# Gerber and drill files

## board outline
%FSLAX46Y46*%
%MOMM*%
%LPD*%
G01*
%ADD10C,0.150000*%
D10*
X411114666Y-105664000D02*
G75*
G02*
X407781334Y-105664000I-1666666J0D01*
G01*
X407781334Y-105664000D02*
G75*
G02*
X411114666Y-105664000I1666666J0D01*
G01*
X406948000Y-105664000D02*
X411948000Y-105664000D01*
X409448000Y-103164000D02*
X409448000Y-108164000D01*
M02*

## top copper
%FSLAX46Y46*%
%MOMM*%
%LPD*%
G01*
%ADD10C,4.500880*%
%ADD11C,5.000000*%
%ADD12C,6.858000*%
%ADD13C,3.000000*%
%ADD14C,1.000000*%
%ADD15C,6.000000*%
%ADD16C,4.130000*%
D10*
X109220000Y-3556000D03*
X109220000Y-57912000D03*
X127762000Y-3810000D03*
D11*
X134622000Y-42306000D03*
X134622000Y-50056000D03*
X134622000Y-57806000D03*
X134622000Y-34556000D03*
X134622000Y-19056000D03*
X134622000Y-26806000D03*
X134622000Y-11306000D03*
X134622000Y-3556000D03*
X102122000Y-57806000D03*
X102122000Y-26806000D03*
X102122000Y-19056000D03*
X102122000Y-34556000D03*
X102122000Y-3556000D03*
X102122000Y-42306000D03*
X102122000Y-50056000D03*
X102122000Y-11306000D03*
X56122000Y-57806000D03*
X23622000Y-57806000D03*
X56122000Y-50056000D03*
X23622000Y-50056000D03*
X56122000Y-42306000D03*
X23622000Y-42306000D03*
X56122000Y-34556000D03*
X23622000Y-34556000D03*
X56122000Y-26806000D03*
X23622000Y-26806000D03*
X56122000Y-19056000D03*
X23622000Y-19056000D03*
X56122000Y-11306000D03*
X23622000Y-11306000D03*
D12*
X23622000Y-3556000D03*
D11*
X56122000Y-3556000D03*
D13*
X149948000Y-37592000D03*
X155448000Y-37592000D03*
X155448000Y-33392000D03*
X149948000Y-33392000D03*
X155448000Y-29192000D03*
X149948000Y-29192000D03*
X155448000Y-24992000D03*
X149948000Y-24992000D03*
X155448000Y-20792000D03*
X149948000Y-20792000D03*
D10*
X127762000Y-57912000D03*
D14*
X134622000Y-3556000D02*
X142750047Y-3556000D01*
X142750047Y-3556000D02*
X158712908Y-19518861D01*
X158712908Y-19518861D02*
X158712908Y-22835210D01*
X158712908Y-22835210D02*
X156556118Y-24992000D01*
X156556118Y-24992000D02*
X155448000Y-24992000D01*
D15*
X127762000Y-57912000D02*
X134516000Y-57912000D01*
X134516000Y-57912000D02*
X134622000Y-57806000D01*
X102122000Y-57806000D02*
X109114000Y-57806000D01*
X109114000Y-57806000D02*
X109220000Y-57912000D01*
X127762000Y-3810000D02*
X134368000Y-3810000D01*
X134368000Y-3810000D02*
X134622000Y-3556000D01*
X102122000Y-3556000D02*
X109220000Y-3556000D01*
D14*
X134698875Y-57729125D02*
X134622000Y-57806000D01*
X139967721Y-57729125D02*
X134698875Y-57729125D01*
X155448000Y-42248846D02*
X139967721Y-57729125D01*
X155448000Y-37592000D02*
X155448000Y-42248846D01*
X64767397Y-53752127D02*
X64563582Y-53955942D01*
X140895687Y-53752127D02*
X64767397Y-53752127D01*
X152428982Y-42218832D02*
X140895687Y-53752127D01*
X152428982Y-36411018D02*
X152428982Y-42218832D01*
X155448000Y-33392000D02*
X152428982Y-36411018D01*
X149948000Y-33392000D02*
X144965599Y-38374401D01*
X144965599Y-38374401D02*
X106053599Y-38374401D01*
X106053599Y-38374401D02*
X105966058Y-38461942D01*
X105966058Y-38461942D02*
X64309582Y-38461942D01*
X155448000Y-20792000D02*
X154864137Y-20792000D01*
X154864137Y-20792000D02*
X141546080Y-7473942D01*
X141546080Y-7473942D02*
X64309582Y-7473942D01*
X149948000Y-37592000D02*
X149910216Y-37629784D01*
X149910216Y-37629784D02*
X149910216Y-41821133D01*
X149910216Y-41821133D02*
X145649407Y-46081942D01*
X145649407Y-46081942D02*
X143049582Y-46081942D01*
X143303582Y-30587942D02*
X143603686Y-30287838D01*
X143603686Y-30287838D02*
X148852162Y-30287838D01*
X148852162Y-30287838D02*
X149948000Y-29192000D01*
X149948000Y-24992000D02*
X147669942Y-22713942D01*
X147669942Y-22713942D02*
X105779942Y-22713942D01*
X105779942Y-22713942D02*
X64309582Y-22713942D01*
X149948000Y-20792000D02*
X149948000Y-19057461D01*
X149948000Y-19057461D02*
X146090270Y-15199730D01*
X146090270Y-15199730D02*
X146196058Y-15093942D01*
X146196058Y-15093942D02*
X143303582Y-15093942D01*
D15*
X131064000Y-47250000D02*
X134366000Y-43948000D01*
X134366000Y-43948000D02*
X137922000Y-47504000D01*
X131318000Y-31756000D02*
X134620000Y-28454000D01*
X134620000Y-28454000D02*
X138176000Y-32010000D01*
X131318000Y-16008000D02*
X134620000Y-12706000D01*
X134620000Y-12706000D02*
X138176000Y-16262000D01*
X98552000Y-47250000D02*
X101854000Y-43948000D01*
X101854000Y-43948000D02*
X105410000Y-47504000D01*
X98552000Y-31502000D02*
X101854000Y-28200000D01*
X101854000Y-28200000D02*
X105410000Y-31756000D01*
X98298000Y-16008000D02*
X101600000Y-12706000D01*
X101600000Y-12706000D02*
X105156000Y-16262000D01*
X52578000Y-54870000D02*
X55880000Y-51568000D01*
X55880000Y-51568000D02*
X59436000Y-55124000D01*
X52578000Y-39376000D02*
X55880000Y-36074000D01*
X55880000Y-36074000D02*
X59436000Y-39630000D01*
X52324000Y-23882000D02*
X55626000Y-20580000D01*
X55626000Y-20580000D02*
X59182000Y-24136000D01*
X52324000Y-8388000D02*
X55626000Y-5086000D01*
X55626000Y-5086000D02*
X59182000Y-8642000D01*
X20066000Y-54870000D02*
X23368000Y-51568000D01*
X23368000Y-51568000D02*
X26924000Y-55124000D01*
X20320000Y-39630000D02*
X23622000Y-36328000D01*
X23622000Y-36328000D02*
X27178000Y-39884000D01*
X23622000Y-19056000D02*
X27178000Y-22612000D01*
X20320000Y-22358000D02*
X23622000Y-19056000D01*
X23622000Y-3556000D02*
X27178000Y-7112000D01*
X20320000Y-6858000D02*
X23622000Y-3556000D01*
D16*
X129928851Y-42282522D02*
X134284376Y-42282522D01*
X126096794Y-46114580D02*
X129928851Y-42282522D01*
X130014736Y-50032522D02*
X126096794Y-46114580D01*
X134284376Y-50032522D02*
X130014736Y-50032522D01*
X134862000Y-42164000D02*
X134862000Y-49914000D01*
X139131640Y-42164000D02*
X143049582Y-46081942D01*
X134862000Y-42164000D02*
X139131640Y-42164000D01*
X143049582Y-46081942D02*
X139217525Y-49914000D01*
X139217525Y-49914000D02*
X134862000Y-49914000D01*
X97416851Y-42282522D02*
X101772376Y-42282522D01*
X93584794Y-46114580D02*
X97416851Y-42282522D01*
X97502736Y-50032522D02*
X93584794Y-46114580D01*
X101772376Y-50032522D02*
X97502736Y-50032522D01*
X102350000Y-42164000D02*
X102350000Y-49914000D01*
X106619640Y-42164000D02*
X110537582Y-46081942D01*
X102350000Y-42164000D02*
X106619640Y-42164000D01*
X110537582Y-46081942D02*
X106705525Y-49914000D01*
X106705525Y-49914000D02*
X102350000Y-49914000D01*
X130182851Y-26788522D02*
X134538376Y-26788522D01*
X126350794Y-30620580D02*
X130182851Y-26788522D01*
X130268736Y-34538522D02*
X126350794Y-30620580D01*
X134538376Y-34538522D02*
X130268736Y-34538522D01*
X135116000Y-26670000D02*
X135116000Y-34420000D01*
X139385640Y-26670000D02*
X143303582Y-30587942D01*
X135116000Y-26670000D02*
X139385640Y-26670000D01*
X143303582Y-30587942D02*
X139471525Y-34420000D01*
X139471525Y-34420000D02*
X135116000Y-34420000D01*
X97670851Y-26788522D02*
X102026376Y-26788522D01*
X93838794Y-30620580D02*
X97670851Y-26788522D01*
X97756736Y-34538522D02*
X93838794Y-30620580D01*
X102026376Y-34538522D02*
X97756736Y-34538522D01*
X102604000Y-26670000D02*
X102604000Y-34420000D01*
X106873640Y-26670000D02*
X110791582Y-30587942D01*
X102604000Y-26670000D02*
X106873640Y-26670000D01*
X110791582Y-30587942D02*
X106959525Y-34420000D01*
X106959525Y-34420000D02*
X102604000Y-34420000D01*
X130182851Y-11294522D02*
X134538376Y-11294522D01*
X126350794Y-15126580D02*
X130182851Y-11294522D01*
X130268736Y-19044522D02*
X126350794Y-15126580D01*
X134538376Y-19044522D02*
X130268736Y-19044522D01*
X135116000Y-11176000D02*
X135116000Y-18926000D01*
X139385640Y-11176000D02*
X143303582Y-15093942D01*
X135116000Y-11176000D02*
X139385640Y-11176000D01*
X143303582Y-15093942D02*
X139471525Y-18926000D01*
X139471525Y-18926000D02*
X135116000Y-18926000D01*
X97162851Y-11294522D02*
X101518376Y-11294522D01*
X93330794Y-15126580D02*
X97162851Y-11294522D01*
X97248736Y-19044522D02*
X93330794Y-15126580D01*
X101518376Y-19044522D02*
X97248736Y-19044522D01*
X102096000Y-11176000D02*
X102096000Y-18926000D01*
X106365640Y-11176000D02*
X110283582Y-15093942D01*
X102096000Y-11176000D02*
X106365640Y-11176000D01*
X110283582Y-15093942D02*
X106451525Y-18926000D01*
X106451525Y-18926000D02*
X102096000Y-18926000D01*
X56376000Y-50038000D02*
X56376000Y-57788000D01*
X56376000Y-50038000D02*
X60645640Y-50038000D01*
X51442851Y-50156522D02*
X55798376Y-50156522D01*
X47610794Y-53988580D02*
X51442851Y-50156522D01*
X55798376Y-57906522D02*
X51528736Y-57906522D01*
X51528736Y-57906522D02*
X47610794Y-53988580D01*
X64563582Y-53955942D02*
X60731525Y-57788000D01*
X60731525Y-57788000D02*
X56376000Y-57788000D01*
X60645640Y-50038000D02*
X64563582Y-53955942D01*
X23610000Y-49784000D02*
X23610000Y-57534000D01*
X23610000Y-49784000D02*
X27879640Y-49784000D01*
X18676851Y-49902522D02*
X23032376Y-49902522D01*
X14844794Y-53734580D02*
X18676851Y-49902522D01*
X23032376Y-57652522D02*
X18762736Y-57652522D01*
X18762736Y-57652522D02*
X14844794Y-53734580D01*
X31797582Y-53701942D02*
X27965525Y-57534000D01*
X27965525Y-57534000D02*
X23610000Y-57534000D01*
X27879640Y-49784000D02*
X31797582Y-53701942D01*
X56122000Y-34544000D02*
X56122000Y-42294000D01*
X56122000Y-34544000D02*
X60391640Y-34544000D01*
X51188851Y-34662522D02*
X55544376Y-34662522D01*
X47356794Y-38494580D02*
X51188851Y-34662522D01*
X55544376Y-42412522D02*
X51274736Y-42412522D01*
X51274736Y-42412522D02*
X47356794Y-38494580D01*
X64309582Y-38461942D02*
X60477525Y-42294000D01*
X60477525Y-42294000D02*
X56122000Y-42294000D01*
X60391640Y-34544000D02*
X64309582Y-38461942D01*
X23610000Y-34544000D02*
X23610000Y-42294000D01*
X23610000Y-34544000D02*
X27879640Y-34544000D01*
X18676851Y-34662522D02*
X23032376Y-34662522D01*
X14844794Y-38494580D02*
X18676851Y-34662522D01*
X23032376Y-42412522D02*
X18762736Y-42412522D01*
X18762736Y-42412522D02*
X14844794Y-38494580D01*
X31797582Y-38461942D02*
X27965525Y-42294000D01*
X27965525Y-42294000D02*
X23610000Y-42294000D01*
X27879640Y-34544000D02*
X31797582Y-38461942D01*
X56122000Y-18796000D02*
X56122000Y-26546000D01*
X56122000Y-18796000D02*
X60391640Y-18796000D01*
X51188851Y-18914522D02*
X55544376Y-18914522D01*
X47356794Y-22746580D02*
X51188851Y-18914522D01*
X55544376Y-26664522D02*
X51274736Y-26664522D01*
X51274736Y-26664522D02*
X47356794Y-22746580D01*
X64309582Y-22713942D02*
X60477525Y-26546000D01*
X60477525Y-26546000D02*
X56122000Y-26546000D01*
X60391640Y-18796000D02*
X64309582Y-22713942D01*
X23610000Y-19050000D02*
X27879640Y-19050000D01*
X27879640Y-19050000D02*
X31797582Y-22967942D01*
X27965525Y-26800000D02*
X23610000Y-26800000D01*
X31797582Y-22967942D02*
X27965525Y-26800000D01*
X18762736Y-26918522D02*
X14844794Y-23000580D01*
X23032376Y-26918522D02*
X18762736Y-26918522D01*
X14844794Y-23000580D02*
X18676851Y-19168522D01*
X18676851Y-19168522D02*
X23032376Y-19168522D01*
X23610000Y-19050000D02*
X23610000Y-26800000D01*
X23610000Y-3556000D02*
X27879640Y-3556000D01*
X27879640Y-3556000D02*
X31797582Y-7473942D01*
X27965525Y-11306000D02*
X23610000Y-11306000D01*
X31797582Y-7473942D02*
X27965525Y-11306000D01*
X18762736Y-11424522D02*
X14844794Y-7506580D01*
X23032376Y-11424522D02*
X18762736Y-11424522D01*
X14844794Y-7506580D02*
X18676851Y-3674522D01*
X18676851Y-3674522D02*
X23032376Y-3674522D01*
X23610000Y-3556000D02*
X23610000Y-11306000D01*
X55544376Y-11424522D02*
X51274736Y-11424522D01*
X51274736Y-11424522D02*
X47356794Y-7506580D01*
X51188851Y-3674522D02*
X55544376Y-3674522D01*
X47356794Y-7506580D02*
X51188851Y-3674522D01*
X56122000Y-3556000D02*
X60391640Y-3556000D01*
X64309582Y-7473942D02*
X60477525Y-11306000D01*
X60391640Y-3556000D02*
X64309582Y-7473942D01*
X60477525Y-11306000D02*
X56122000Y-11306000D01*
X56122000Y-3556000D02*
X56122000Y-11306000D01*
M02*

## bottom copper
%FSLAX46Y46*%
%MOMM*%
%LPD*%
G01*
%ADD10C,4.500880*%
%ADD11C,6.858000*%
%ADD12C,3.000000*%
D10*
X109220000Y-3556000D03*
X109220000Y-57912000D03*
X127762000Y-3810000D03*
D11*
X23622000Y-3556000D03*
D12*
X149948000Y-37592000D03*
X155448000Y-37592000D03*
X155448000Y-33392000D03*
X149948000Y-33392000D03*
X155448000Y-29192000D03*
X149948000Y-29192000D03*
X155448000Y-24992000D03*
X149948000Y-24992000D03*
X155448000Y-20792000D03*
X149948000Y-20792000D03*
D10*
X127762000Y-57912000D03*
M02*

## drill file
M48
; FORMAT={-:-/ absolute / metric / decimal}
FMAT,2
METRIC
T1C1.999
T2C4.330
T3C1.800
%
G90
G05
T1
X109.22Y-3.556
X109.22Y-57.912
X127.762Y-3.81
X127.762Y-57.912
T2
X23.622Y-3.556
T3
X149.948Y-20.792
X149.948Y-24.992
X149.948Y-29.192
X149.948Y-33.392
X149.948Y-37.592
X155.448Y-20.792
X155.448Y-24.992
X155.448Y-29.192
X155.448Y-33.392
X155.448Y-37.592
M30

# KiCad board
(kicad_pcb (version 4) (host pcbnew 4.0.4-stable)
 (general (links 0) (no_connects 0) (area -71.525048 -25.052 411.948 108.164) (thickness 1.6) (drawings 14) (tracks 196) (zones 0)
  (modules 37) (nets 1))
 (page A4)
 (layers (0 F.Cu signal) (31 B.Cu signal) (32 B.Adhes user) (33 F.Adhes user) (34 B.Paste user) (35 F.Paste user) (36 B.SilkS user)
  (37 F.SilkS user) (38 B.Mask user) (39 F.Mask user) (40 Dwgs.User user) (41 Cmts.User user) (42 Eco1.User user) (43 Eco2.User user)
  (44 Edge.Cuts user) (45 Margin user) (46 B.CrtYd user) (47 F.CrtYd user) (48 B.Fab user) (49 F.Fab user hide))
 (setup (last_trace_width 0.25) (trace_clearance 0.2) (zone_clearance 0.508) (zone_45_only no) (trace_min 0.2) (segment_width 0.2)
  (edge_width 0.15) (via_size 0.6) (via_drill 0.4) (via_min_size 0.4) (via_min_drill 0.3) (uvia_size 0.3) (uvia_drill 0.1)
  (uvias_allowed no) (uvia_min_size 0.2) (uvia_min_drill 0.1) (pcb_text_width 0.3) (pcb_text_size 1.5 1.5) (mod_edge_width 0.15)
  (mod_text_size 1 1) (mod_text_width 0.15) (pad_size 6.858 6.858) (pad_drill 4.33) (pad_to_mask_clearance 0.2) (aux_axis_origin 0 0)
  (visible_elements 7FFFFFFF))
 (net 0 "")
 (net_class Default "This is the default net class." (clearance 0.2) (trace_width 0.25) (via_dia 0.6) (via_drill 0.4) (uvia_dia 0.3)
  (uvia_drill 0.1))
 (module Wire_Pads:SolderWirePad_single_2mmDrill (layer F.Cu) (at 109.22 3.556)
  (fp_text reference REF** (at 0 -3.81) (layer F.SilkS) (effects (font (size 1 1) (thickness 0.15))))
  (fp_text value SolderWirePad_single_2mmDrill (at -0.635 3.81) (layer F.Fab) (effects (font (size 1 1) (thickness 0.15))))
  (pad 1 thru_hole circle (at 0 0) (size 4.50088 4.50088) (drill 1.99898) (layers *.Cu *.Mask)))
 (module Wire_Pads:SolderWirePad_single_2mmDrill (layer F.Cu) (at 109.22 57.912)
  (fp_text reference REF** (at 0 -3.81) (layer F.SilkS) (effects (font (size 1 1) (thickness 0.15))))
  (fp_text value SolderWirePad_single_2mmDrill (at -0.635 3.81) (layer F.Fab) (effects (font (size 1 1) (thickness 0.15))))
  (pad 1 thru_hole circle (at 0 0) (size 4.50088 4.50088) (drill 1.99898) (layers *.Cu *.Mask)))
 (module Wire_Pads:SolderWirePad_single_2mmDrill (layer F.Cu) (at 127.762 3.81)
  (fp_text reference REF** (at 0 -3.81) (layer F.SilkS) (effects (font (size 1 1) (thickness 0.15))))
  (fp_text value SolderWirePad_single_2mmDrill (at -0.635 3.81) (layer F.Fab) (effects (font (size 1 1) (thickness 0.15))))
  (pad 1 thru_hole circle (at 0 0) (size 4.50088 4.50088) (drill 1.99898) (layers *.Cu *.Mask)))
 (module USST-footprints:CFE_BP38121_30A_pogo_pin (layer F.Cu) (at 174.5 53.736)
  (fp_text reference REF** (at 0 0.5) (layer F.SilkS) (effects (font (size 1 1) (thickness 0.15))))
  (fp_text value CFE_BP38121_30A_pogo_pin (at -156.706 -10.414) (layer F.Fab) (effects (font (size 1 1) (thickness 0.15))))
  (pad 6 smd circle (at -39.878 -11.43) (size 5 5) (layers F.Cu F.Paste F.Mask)))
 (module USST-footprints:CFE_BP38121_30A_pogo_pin (layer F.Cu) (at 174.5 61.486)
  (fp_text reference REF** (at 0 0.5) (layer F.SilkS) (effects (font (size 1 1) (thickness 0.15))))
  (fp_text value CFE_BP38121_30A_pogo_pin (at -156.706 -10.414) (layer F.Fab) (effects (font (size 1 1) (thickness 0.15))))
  (pad 7 smd circle (at -39.878 -11.43) (size 5 5) (layers F.Cu F.Paste F.Mask)))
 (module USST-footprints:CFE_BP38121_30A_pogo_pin (layer F.Cu) (at 174.5 69.236)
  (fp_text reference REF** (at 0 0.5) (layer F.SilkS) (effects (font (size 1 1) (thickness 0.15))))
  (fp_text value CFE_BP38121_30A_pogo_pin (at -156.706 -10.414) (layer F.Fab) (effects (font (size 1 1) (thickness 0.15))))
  (pad 8 smd circle (at -39.878 -11.43) (size 5 5) (layers F.Cu F.Paste F.Mask)))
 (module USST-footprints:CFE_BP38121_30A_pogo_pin (layer F.Cu) (at 174.5 45.986)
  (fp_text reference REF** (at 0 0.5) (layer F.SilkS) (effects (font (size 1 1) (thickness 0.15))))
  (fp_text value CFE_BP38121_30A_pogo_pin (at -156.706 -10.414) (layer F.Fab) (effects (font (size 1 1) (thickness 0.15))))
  (pad 5 smd circle (at -39.878 -11.43) (size 5 5) (layers F.Cu F.Paste F.Mask)))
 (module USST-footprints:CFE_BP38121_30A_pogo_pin (layer F.Cu) (at 174.5 30.486)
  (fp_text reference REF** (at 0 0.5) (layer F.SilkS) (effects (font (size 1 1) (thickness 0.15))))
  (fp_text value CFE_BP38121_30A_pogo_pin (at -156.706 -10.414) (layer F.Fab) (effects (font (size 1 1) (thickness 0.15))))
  (pad 3 smd circle (at -39.878 -11.43) (size 5 5) (layers F.Cu F.Paste F.Mask)))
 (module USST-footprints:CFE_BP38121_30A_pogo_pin (layer F.Cu) (at 174.5 38.236)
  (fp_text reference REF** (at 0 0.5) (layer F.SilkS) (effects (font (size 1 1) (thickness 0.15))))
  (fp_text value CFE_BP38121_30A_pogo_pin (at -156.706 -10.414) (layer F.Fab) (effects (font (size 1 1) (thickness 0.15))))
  (pad 4 smd circle (at -39.878 -11.43) (size 5 5) (layers F.Cu F.Paste F.Mask)))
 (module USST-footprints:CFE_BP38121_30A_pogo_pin (layer F.Cu) (at 174.5 22.736)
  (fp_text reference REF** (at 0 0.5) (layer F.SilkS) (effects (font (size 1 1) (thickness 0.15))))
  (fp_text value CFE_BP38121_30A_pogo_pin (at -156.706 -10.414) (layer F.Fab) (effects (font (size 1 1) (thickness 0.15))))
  (pad 2 smd circle (at -39.878 -11.43) (size 5 5) (layers F.Cu F.Paste F.Mask)))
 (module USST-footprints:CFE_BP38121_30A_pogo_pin (layer F.Cu) (at 174.5 14.986)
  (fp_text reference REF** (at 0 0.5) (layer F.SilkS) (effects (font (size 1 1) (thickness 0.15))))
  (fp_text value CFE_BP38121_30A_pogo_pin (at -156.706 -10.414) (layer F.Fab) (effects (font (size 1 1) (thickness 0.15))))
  (pad 1 smd circle (at -39.878 -11.43) (size 5 5) (layers F.Cu F.Paste F.Mask)))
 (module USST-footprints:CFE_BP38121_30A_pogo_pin (layer F.Cu) (at 142 69.236)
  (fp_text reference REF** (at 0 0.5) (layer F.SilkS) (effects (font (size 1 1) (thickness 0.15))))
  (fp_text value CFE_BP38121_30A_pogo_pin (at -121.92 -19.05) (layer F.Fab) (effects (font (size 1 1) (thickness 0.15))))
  (pad 8 smd circle (at -39.878 -11.43) (size 5 5) (layers F.Cu F.Paste F.Mask)))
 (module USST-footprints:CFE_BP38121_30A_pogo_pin (layer F.Cu) (at 142 38.236)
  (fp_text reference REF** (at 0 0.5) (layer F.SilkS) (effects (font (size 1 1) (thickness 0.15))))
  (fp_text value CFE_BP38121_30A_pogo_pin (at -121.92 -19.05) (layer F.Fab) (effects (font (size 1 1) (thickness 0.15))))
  (pad 4 smd circle (at -39.878 -11.43) (size 5 5) (layers F.Cu F.Paste F.Mask)))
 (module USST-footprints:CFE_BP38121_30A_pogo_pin (layer F.Cu) (at 142 30.486)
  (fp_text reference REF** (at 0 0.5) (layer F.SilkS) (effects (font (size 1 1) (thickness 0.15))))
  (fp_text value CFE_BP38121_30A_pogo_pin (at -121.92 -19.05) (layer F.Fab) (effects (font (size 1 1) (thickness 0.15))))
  (pad 3 smd circle (at -39.878 -11.43) (size 5 5) (layers F.Cu F.Paste F.Mask)))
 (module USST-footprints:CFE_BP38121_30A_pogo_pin (layer F.Cu) (at 142 45.986)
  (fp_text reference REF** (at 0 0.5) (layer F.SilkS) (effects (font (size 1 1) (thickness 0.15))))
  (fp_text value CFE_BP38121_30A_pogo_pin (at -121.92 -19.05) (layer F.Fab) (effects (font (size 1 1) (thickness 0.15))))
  (pad 5 smd circle (at -39.878 -11.43) (size 5 5) (layers F.Cu F.Paste F.Mask)))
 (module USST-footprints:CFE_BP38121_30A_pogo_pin (layer F.Cu) (at 142 14.986)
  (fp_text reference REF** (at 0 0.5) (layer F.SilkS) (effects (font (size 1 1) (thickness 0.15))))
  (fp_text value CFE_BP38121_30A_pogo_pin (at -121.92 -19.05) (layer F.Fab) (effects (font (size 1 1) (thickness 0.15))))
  (pad 1 smd circle (at -39.878 -11.43) (size 5 5) (layers F.Cu F.Paste F.Mask)))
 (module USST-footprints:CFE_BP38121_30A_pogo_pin (layer F.Cu) (at 142 53.736)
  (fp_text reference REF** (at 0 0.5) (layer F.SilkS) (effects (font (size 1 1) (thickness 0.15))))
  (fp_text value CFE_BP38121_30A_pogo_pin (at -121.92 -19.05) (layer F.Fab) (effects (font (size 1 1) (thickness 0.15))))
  (pad 6 smd circle (at -39.878 -11.43) (size 5 5) (layers F.Cu F.Paste F.Mask)))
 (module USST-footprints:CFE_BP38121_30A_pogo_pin (layer F.Cu) (at 142 61.486)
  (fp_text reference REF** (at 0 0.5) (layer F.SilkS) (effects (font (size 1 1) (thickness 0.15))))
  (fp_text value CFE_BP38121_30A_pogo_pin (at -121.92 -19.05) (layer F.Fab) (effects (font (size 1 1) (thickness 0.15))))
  (pad 7 smd circle (at -39.878 -11.43) (size 5 5) (layers F.Cu F.Paste F.Mask)))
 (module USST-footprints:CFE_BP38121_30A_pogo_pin (layer F.Cu) (at 142 22.736)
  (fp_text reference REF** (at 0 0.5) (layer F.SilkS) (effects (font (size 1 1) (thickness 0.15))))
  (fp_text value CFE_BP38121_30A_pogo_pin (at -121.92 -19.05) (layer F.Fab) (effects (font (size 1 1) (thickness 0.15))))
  (pad 2 smd circle (at -39.878 -11.43) (size 5 5) (layers F.Cu F.Paste F.Mask)))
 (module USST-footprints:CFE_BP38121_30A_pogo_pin (layer F.Cu) (at 96 69.236)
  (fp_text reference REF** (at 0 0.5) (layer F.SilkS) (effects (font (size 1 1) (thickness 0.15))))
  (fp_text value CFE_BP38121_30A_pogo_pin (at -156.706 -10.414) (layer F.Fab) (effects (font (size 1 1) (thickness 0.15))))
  (pad 8 smd circle (at -39.878 -11.43) (size 5 5) (layers F.Cu F.Paste F.Mask)))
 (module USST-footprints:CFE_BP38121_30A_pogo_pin (layer F.Cu) (at 63.5 69.236)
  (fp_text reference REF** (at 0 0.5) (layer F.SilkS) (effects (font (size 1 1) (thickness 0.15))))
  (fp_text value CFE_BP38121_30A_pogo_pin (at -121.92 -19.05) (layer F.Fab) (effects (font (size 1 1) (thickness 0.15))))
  (pad 8 smd circle (at -39.878 -11.43) (size 5 5) (layers F.Cu F.Paste F.Mask)))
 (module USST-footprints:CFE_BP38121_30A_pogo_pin (layer F.Cu) (at 96 61.486)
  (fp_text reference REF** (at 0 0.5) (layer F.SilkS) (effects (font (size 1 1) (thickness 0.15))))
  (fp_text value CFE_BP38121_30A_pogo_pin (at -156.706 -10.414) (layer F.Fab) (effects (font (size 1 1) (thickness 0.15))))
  (pad 7 smd circle (at -39.878 -11.43) (size 5 5) (layers F.Cu F.Paste F.Mask)))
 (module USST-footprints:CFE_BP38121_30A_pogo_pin (layer F.Cu) (at 63.5 61.486)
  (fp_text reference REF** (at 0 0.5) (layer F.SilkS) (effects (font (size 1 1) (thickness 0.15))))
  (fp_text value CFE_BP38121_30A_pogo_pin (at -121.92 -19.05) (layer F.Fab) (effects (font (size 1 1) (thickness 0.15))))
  (pad 7 smd circle (at -39.878 -11.43) (size 5 5) (layers F.Cu F.Paste F.Mask)))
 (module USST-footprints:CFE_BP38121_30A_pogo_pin (layer F.Cu) (at 96 53.736)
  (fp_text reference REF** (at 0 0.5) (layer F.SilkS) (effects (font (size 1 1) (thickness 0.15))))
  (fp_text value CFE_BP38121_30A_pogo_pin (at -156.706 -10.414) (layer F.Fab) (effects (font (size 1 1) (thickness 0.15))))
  (pad 6 smd circle (at -39.878 -11.43) (size 5 5) (layers F.Cu F.Paste F.Mask)))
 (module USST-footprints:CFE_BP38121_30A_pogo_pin (layer F.Cu) (at 63.5 53.736)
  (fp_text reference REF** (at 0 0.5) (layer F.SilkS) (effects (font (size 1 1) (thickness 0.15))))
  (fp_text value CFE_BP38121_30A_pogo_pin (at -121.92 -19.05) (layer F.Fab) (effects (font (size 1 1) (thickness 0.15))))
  (pad 6 smd circle (at -39.878 -11.43) (size 5 5) (layers F.Cu F.Paste F.Mask)))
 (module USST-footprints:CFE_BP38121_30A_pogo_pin (layer F.Cu) (at 96 45.986)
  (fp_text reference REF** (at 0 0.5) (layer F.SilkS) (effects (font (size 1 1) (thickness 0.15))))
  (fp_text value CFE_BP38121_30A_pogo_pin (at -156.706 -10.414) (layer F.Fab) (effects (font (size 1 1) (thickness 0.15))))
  (pad 5 smd circle (at -39.878 -11.43) (size 5 5) (layers F.Cu F.Paste F.Mask)))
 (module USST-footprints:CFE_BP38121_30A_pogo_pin (layer F.Cu) (at 63.5 45.986)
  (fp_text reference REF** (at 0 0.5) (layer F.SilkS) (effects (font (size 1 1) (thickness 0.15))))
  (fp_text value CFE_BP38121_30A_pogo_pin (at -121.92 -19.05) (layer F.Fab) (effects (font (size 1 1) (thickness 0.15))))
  (pad 5 smd circle (at -39.878 -11.43) (size 5 5) (layers F.Cu F.Paste F.Mask)))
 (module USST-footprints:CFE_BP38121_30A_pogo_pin (layer F.Cu) (at 96 38.236)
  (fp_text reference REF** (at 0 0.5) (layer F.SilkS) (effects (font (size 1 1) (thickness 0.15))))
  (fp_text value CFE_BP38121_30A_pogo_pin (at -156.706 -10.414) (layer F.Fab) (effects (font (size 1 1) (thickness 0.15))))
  (pad 4 smd circle (at -39.878 -11.43) (size 5 5) (layers F.Cu F.Paste F.Mask)))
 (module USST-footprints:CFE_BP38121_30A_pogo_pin (layer F.Cu) (at 63.5 38.236)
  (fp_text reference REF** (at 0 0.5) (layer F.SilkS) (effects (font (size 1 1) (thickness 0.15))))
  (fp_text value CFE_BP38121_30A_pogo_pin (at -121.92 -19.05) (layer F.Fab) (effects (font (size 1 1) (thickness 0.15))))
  (pad 4 smd circle (at -39.878 -11.43) (size 5 5) (layers F.Cu F.Paste F.Mask)))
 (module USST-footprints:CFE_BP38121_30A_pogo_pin (layer F.Cu) (at 96 30.486)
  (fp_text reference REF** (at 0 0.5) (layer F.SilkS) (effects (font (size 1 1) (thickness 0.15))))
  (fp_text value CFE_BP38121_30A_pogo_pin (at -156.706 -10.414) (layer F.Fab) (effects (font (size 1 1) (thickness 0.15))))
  (pad 3 smd circle (at -39.878 -11.43) (size 5 5) (layers F.Cu F.Paste F.Mask)))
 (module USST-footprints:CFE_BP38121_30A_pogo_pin (layer F.Cu) (at 63.5 30.486)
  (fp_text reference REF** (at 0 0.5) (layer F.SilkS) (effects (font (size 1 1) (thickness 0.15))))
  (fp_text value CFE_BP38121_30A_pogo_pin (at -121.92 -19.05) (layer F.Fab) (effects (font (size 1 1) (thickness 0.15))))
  (pad 3 smd circle (at -39.878 -11.43) (size 5 5) (layers F.Cu F.Paste F.Mask)))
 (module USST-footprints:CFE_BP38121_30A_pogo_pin (layer F.Cu) (at 96 22.736)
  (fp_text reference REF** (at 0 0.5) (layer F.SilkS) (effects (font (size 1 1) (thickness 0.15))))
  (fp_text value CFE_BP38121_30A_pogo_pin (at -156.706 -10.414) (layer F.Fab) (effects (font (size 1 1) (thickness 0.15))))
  (pad 2 smd circle (at -39.878 -11.43) (size 5 5) (layers F.Cu F.Paste F.Mask)))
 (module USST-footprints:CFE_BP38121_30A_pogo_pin (layer F.Cu) (at 63.5 22.736)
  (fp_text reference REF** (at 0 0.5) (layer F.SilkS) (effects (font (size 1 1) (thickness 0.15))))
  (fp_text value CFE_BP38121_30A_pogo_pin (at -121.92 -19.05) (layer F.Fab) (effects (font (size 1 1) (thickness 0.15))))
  (pad 2 smd circle (at -39.878 -11.43) (size 5 5) (layers F.Cu F.Paste F.Mask)))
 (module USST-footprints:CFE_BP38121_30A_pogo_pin (layer F.Cu) (at 63.5 14.986)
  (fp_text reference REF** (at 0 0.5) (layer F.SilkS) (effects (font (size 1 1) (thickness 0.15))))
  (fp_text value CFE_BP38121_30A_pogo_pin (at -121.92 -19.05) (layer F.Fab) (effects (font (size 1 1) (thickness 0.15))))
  (pad 1 thru_hole circle (at -39.878 -11.43) (size 6.858 6.858) (drill 4.33) (layers *.Cu *.Mask)))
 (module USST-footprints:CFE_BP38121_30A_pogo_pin (layer F.Cu) (at 96 14.986)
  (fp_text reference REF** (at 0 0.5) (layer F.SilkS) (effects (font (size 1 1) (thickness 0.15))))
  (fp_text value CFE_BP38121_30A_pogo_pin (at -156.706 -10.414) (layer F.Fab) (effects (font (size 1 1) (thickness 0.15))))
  (pad 1 smd circle (at -39.878 -11.43) (size 5 5) (layers F.Cu F.Paste F.Mask)))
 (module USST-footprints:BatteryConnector (layer F.Cu) (at 149.948 37.592)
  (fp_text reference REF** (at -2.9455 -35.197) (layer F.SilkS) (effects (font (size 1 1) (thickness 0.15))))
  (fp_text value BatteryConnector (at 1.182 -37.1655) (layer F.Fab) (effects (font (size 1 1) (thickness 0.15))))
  (pad "" np_thru_hole circle (at 0 0) (size 3 3) (drill 1.8) (layers *.Cu))
  (pad "" np_thru_hole circle (at 5.5 0) (size 3 3) (drill 1.8) (layers *.Cu))
  (pad "" np_thru_hole circle (at 5.5 -4.2) (size 3 3) (drill 1.8) (layers *.Cu))
  (pad "" np_thru_hole circle (at 0 -4.2) (size 3 3) (drill 1.8) (layers *.Cu))
  (pad "" np_thru_hole circle (at 5.5 -8.4) (size 3 3) (drill 1.8) (layers *.Cu))
  (pad "" np_thru_hole circle (at 0 -8.4) (size 3 3) (drill 1.8) (layers *.Cu))
  (pad "" np_thru_hole circle (at 5.5 -12.6) (size 3 3) (drill 1.8) (layers *.Cu))
  (pad "" np_thru_hole circle (at 0 -12.6) (size 3 3) (drill 1.8) (layers *.Cu))
  (pad "" np_thru_hole circle (at 5.5 -16.8) (size 3 3) (drill 1.8) (layers *.Cu))
  (pad "" np_thru_hole circle (at 0 -16.8) (size 3 3) (drill 1.8) (layers *.Cu)))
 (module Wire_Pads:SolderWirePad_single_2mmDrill (layer F.Cu) (at 127.762 57.912)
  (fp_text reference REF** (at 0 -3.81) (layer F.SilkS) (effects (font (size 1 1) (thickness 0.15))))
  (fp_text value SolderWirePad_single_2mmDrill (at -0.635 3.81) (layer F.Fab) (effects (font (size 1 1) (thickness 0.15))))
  (pad 1 thru_hole circle (at 0 0) (size 4.50088 4.50088) (drill 1.99898) (layers *.Cu *.Mask)))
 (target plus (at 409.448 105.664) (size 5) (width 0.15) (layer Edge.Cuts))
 (segment (start 134.622 3.556) (end 142.750047 3.556) (width 1) (layer F.Cu) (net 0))
 (segment (start 142.750047 3.556) (end 158.712908 19.518861) (width 1) (layer F.Cu) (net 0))
 (segment (start 158.712908 19.518861) (end 158.712908 22.83521) (width 1) (layer F.Cu) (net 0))
 (segment (start 158.712908 22.83521) (end 156.556118 24.992) (width 1) (layer F.Cu) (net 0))
 (segment (start 156.556118 24.992) (end 155.448 24.992) (width 1) (layer F.Cu) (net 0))
 (segment (start 127.762 57.912) (end 134.516 57.912) (width 6) (layer F.Cu) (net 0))
 (segment (start 134.516 57.912) (end 134.622 57.806) (width 6) (layer F.Cu) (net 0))
 (segment (start 102.122 57.806) (end 109.114 57.806) (width 6) (layer F.Cu) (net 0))
 (segment (start 109.114 57.806) (end 109.22 57.912) (width 6) (layer F.Cu) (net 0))
 (segment (start 127.762 3.81) (end 134.368 3.81) (width 6) (layer F.Cu) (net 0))
 (segment (start 134.368 3.81) (end 134.622 3.556) (width 6) (layer F.Cu) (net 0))
 (segment (start 102.122 3.556) (end 109.22 3.556) (width 6) (layer F.Cu) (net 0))
 (segment (start 134.698875 57.729125) (end 134.622 57.806) (width 1) (layer F.Cu) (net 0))
 (segment (start 139.967721 57.729125) (end 134.698875 57.729125) (width 1) (layer F.Cu) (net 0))
 (segment (start 155.448 42.248846) (end 139.967721 57.729125) (width 1) (layer F.Cu) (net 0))
 (segment (start 155.448 37.592) (end 155.448 42.248846) (width 1) (layer F.Cu) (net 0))
 (segment (start 64.767397 53.752127) (end 64.563582 53.955942) (width 1) (layer F.Cu) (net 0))
 (segment (start 140.895687 53.752127) (end 64.767397 53.752127) (width 1) (layer F.Cu) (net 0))
 (segment (start 152.428982 42.218832) (end 140.895687 53.752127) (width 1) (layer F.Cu) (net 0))
 (segment (start 152.428982 36.411018) (end 152.428982 42.218832) (width 1) (layer F.Cu) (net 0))
 (segment (start 155.448 33.392) (end 152.428982 36.411018) (width 1) (layer F.Cu) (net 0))
 (segment (start 149.948 33.392) (end 144.965599 38.374401) (width 1) (layer F.Cu) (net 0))
 (segment (start 144.965599 38.374401) (end 106.053599 38.374401) (width 1) (layer F.Cu) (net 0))
 (segment (start 106.053599 38.374401) (end 105.966058 38.461942) (width 1) (layer F.Cu) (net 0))
 (segment (start 105.966058 38.461942) (end 64.309582 38.461942) (width 1) (layer F.Cu) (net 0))
 (segment (start 155.448 20.792) (end 154.864137 20.792) (width 1) (layer F.Cu) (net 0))
 (segment (start 154.864137 20.792) (end 141.54608 7.473942) (width 1) (layer F.Cu) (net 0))
 (segment (start 141.54608 7.473942) (end 64.309582 7.473942) (width 1) (layer F.Cu) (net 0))
 (segment (start 149.948 37.592) (end 149.910216 37.629784) (width 1) (layer F.Cu) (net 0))
 (segment (start 149.910216 37.629784) (end 149.910216 41.821133) (width 1) (layer F.Cu) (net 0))
 (segment (start 149.910216 41.821133) (end 145.649407 46.081942) (width 1) (layer F.Cu) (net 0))
 (segment (start 145.649407 46.081942) (end 143.049582 46.081942) (width 1) (layer F.Cu) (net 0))
 (segment (start 143.303582 30.587942) (end 143.603686 30.287838) (width 1) (layer F.Cu) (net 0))
 (segment (start 143.603686 30.287838) (end 148.852162 30.287838) (width 1) (layer F.Cu) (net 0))
 (segment (start 148.852162 30.287838) (end 149.948 29.192) (width 1) (layer F.Cu) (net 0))
 (segment (start 149.948 24.992) (end 147.669942 22.713942) (width 1) (layer F.Cu) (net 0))
 (segment (start 147.669942 22.713942) (end 105.779942 22.713942) (width 1) (layer F.Cu) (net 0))
 (segment (start 105.779942 22.713942) (end 64.309582 22.713942) (width 1) (layer F.Cu) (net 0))
 (segment (start 149.948 20.792) (end 149.948 19.057461) (width 1) (layer F.Cu) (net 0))
 (segment (start 149.948 19.057461) (end 146.09027 15.19973) (width 1) (layer F.Cu) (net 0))
 (segment (start 146.09027 15.19973) (end 146.196058 15.093942) (width 1) (layer F.Cu) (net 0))
 (segment (start 146.196058 15.093942) (end 143.303582 15.093942) (width 1) (layer F.Cu) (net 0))
 (segment (start 131.064 47.25) (end 134.366 43.948) (width 6) (layer F.Cu) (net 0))
 (segment (start 134.366 43.948) (end 137.922 47.504) (width 6) (layer F.Cu) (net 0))
 (segment (start 131.318 31.756) (end 134.62 28.454) (width 6) (layer F.Cu) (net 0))
 (segment (start 134.62 28.454) (end 138.176 32.01) (width 6) (layer F.Cu) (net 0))
 (segment (start 131.318 16.008) (end 134.62 12.706) (width 6) (layer F.Cu) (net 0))
 (segment (start 134.62 12.706) (end 138.176 16.262) (width 6) (layer F.Cu) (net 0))
 (segment (start 98.552 47.25) (end 101.854 43.948) (width 6) (layer F.Cu) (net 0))
 (segment (start 101.854 43.948) (end 105.41 47.504) (width 6) (layer F.Cu) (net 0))
 (segment (start 98.552 31.502) (end 101.854 28.2) (width 6) (layer F.Cu) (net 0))
 (segment (start 101.854 28.2) (end 105.41 31.756) (width 6) (layer F.Cu) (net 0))
 (segment (start 98.298 16.008) (end 101.6 12.706) (width 6) (layer F.Cu) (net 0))
 (segment (start 101.6 12.706) (end 105.156 16.262) (width 6) (layer F.Cu) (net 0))
 (segment (start 52.578 54.87) (end 55.88 51.568) (width 6) (layer F.Cu) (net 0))
 (segment (start 55.88 51.568) (end 59.436 55.124) (width 6) (layer F.Cu) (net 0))
 (segment (start 52.578 39.376) (end 55.88 36.074) (width 6) (layer F.Cu) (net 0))
 (segment (start 55.88 36.074) (end 59.436 39.63) (width 6) (layer F.Cu) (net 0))
 (segment (start 52.324 23.882) (end 55.626 20.58) (width 6) (layer F.Cu) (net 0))
 (segment (start 55.626 20.58) (end 59.182 24.136) (width 6) (layer F.Cu) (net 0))
 (segment (start 52.324 8.388) (end 55.626 5.086) (width 6) (layer F.Cu) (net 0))
 (segment (start 55.626 5.086) (end 59.182 8.642) (width 6) (layer F.Cu) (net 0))
 (segment (start 20.066 54.87) (end 23.368 51.568) (width 6) (layer F.Cu) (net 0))
 (segment (start 23.368 51.568) (end 26.924 55.124) (width 6) (layer F.Cu) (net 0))
 (segment (start 20.32 39.63) (end 23.622 36.328) (width 6) (layer F.Cu) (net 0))
 (segment (start 23.622 36.328) (end 27.178 39.884) (width 6) (layer F.Cu) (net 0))
 (segment (start 23.622 19.056) (end 27.178 22.612) (width 6) (layer F.Cu) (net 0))
 (segment (start 20.32 22.358) (end 23.622 19.056) (width 6) (layer F.Cu) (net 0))
 (segment (start 23.622 3.556) (end 27.178 7.112) (width 6) (layer F.Cu) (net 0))
 (segment (start 20.32 6.858) (end 23.622 3.556) (width 6) (layer F.Cu) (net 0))
 (segment (start 129.928851 42.282522) (end 134.284376 42.282522) (width 4.13) (layer F.Cu) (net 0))
 (segment (start 126.096794 46.11458) (end 129.928851 42.282522) (width 4.13) (layer F.Cu) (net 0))
 (segment (start 130.014736 50.032522) (end 126.096794 46.11458) (width 4.13) (layer F.Cu) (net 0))
 (segment (start 134.284376 50.032522) (end 130.014736 50.032522) (width 4.13) (layer F.Cu) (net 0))
 (segment (start 134.862 42.164) (end 134.862 49.914) (width 4.13) (layer F.Cu) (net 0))
 (segment (start 139.13164 42.164) (end 143.049582 46.081942) (width 4.13) (layer F.Cu) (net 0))
 (segment (start 134.862 42.164) (end 139.13164 42.164) (width 4.13) (layer F.Cu) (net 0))
 (segment (start 143.049582 46.081942) (end 139.217525 49.914) (width 4.13) (layer F.Cu) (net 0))
 (segment (start 139.217525 49.914) (end 134.862 49.914) (width 4.13) (layer F.Cu) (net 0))
 (segment (start 97.416851 42.282522) (end 101.772376 42.282522) (width 4.13) (layer F.Cu) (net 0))
 (segment (start 93.584794 46.11458) (end 97.416851 42.282522) (width 4.13) (layer F.Cu) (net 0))
 (segment (start 97.502736 50.032522) (end 93.584794 46.11458) (width 4.13) (layer F.Cu) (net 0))
 (segment (start 101.772376 50.032522) (end 97.502736 50.032522) (width 4.13) (layer F.Cu) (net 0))
 (segment (start 102.35 42.164) (end 102.35 49.914) (width 4.13) (layer F.Cu) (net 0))
 (segment (start 106.61964 42.164) (end 110.537582 46.081942) (width 4.13) (layer F.Cu) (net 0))
 (segment (start 102.35 42.164) (end 106.61964 42.164) (width 4.13) (layer F.Cu) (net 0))
 (segment (start 110.537582 46.081942) (end 106.705525 49.914) (width 4.13) (layer F.Cu) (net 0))
 (segment (start 106.705525 49.914) (end 102.35 49.914) (width 4.13) (layer F.Cu) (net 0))
 (segment (start 130.182851 26.788522) (end 134.538376 26.788522) (width 4.13) (layer F.Cu) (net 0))
 (segment (start 126.350794 30.62058) (end 130.182851 26.788522) (width 4.13) (layer F.Cu) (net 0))
 (segment (start 130.268736 34.538522) (end 126.350794 30.62058) (width 4.13) (layer F.Cu) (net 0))
 (segment (start 134.538376 34.538522) (end 130.268736 34.538522) (width 4.13) (layer F.Cu) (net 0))
 (segment (start 135.116 26.67) (end 135.116 34.42) (width 4.13) (layer F.Cu) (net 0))
 (segment (start 139.38564 26.67) (end 143.303582 30.587942) (width 4.13) (layer F.Cu) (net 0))
 (segment (start 135.116 26.67) (end 139.38564 26.67) (width 4.13) (layer F.Cu) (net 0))
 (segment (start 143.303582 30.587942) (end 139.471525 34.42) (width 4.13) (layer F.Cu) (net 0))
 (segment (start 139.471525 34.42) (end 135.116 34.42) (width 4.13) (layer F.Cu) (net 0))
 (segment (start 97.670851 26.788522) (end 102.026376 26.788522) (width 4.13) (layer F.Cu) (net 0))
 (segment (start 93.838794 30.62058) (end 97.670851 26.788522) (width 4.13) (layer F.Cu) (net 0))
 (segment (start 97.756736 34.538522) (end 93.838794 30.62058) (width 4.13) (layer F.Cu) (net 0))
 (segment (start 102.026376 34.538522) (end 97.756736 34.538522) (width 4.13) (layer F.Cu) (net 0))
 (segment (start 102.604 26.67) (end 102.604 34.42) (width 4.13) (layer F.Cu) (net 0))
 (segment (start 106.87364 26.67) (end 110.791582 30.587942) (width 4.13) (layer F.Cu) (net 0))
 (segment (start 102.604 26.67) (end 106.87364 26.67) (width 4.13) (layer F.Cu) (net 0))
 (segment (start 110.791582 30.587942) (end 106.959525 34.42) (width 4.13) (layer F.Cu) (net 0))
 (segment (start 106.959525 34.42) (end 102.604 34.42) (width 4.13) (layer F.Cu) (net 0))
 (segment (start 130.182851 11.294522) (end 134.538376 11.294522) (width 4.13) (layer F.Cu) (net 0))
 (segment (start 126.350794 15.12658) (end 130.182851 11.294522) (width 4.13) (layer F.Cu) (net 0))
 (segment (start 130.268736 19.044522) (end 126.350794 15.12658) (width 4.13) (layer F.Cu) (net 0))
 (segment (start 134.538376 19.044522) (end 130.268736 19.044522) (width 4.13) (layer F.Cu) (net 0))
 (segment (start 135.116 11.176) (end 135.116 18.926) (width 4.13) (layer F.Cu) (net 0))
 (segment (start 139.38564 11.176) (end 143.303582 15.093942) (width 4.13) (layer F.Cu) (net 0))
 (segment (start 135.116 11.176) (end 139.38564 11.176) (width 4.13) (layer F.Cu) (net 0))
 (segment (start 143.303582 15.093942) (end 139.471525 18.926) (width 4.13) (layer F.Cu) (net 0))
 (segment (start 139.471525 18.926) (end 135.116 18.926) (width 4.13) (layer F.Cu) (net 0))
 (segment (start 97.162851 11.294522) (end 101.518376 11.294522) (width 4.13) (layer F.Cu) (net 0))
 (segment (start 93.330794 15.12658) (end 97.162851 11.294522) (width 4.13) (layer F.Cu) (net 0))
 (segment (start 97.248736 19.044522) (end 93.330794 15.12658) (width 4.13) (layer F.Cu) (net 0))
 (segment (start 101.518376 19.044522) (end 97.248736 19.044522) (width 4.13) (layer F.Cu) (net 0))
 (segment (start 102.096 11.176) (end 102.096 18.926) (width 4.13) (layer F.Cu) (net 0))
 (segment (start 106.36564 11.176) (end 110.283582 15.093942) (width 4.13) (layer F.Cu) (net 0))
 (segment (start 102.096 11.176) (end 106.36564 11.176) (width 4.13) (layer F.Cu) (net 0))
 (segment (start 110.283582 15.093942) (end 106.451525 18.926) (width 4.13) (layer F.Cu) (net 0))
 (segment (start 106.451525 18.926) (end 102.096 18.926) (width 4.13) (layer F.Cu) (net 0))
 (segment (start 56.376 50.038) (end 56.376 57.788) (width 4.13) (layer F.Cu) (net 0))
 (segment (start 56.376 50.038) (end 60.64564 50.038) (width 4.13) (layer F.Cu) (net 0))
 (segment (start 51.442851 50.156522) (end 55.798376 50.156522) (width 4.13) (layer F.Cu) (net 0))
 (segment (start 47.610794 53.98858) (end 51.442851 50.156522) (width 4.13) (layer F.Cu) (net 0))
 (segment (start 55.798376 57.906522) (end 51.528736 57.906522) (width 4.13) (layer F.Cu) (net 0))
 (segment (start 51.528736 57.906522) (end 47.610794 53.98858) (width 4.13) (layer F.Cu) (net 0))
 (segment (start 64.563582 53.955942) (end 60.731525 57.788) (width 4.13) (layer F.Cu) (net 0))
 (segment (start 60.731525 57.788) (end 56.376 57.788) (width 4.13) (layer F.Cu) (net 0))
 (segment (start 60.64564 50.038) (end 64.563582 53.955942) (width 4.13) (layer F.Cu) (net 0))
 (segment (start 23.61 49.784) (end 23.61 57.534) (width 4.13) (layer F.Cu) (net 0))
 (segment (start 23.61 49.784) (end 27.87964 49.784) (width 4.13) (layer F.Cu) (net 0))
 (segment (start 18.676851 49.902522) (end 23.032376 49.902522) (width 4.13) (layer F.Cu) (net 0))
 (segment (start 14.844794 53.73458) (end 18.676851 49.902522) (width 4.13) (layer F.Cu) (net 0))
 (segment (start 23.032376 57.652522) (end 18.762736 57.652522) (width 4.13) (layer F.Cu) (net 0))
 (segment (start 18.762736 57.652522) (end 14.844794 53.73458) (width 4.13) (layer F.Cu) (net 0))
 (segment (start 31.797582 53.701942) (end 27.965525 57.534) (width 4.13) (layer F.Cu) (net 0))
 (segment (start 27.965525 57.534) (end 23.61 57.534) (width 4.13) (layer F.Cu) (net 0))
 (segment (start 27.87964 49.784) (end 31.797582 53.701942) (width 4.13) (layer F.Cu) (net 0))
 (segment (start 56.122 34.544) (end 56.122 42.294) (width 4.13) (layer F.Cu) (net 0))
 (segment (start 56.122 34.544) (end 60.39164 34.544) (width 4.13) (layer F.Cu) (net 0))
 (segment (start 51.188851 34.662522) (end 55.544376 34.662522) (width 4.13) (layer F.Cu) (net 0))
 (segment (start 47.356794 38.49458) (end 51.188851 34.662522) (width 4.13) (layer F.Cu) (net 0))
 (segment (start 55.544376 42.412522) (end 51.274736 42.412522) (width 4.13) (layer F.Cu) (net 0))
 (segment (start 51.274736 42.412522) (end 47.356794 38.49458) (width 4.13) (layer F.Cu) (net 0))
 (segment (start 64.309582 38.461942) (end 60.477525 42.294) (width 4.13) (layer F.Cu) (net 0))
 (segment (start 60.477525 42.294) (end 56.122 42.294) (width 4.13) (layer F.Cu) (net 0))
 (segment (start 60.39164 34.544) (end 64.309582 38.461942) (width 4.13) (layer F.Cu) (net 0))
 (segment (start 23.61 34.544) (end 23.61 42.294) (width 4.13) (layer F.Cu) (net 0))
 (segment (start 23.61 34.544) (end 27.87964 34.544) (width 4.13) (layer F.Cu) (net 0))
 (segment (start 18.676851 34.662522) (end 23.032376 34.662522) (width 4.13) (layer F.Cu) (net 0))
 (segment (start 14.844794 38.49458) (end 18.676851 34.662522) (width 4.13) (layer F.Cu) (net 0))
 (segment (start 23.032376 42.412522) (end 18.762736 42.412522) (width 4.13) (layer F.Cu) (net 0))
 (segment (start 18.762736 42.412522) (end 14.844794 38.49458) (width 4.13) (layer F.Cu) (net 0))
 (segment (start 31.797582 38.461942) (end 27.965525 42.294) (width 4.13) (layer F.Cu) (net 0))
 (segment (start 27.965525 42.294) (end 23.61 42.294) (width 4.13) (layer F.Cu) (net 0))
 (segment (start 27.87964 34.544) (end 31.797582 38.461942) (width 4.13) (layer F.Cu) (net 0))
 (segment (start 56.122 18.796) (end 56.122 26.546) (width 4.13) (layer F.Cu) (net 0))
 (segment (start 56.122 18.796) (end 60.39164 18.796) (width 4.13) (layer F.Cu) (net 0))
 (segment (start 51.188851 18.914522) (end 55.544376 18.914522) (width 4.13) (layer F.Cu) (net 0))
 (segment (start 47.356794 22.74658) (end 51.188851 18.914522) (width 4.13) (layer F.Cu) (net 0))
 (segment (start 55.544376 26.664522) (end 51.274736 26.664522) (width 4.13) (layer F.Cu) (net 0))
 (segment (start 51.274736 26.664522) (end 47.356794 22.74658) (width 4.13) (layer F.Cu) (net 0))
 (segment (start 64.309582 22.713942) (end 60.477525 26.546) (width 4.13) (layer F.Cu) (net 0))
 (segment (start 60.477525 26.546) (end 56.122 26.546) (width 4.13) (layer F.Cu) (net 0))
 (segment (start 60.39164 18.796) (end 64.309582 22.713942) (width 4.13) (layer F.Cu) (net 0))
 (segment (start 23.61 19.05) (end 27.87964 19.05) (width 4.13) (layer F.Cu) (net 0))
 (segment (start 27.87964 19.05) (end 31.797582 22.967942) (width 4.13) (layer F.Cu) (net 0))
 (segment (start 27.965525 26.8) (end 23.61 26.8) (width 4.13) (layer F.Cu) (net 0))
 (segment (start 31.797582 22.967942) (end 27.965525 26.8) (width 4.13) (layer F.Cu) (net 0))
 (segment (start 18.762736 26.918522) (end 14.844794 23.00058) (width 4.13) (layer F.Cu) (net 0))
 (segment (start 23.032376 26.918522) (end 18.762736 26.918522) (width 4.13) (layer F.Cu) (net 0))
 (segment (start 14.844794 23.00058) (end 18.676851 19.168522) (width 4.13) (layer F.Cu) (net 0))
 (segment (start 18.676851 19.168522) (end 23.032376 19.168522) (width 4.13) (layer F.Cu) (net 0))
 (segment (start 23.61 19.05) (end 23.61 26.8) (width 4.13) (layer F.Cu) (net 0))
 (segment (start 23.61 3.556) (end 27.87964 3.556) (width 4.13) (layer F.Cu) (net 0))
 (segment (start 27.87964 3.556) (end 31.797582 7.473942) (width 4.13) (layer F.Cu) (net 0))
 (segment (start 27.965525 11.306) (end 23.61 11.306) (width 4.13) (layer F.Cu) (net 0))
 (segment (start 31.797582 7.473942) (end 27.965525 11.306) (width 4.13) (layer F.Cu) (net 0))
 (segment (start 18.762736 11.424522) (end 14.844794 7.50658) (width 4.13) (layer F.Cu) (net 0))
 (segment (start 23.032376 11.424522) (end 18.762736 11.424522) (width 4.13) (layer F.Cu) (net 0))
 (segment (start 14.844794 7.50658) (end 18.676851 3.674522) (width 4.13) (layer F.Cu) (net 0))
 (segment (start 18.676851 3.674522) (end 23.032376 3.674522) (width 4.13) (layer F.Cu) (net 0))
 (segment (start 23.61 3.556) (end 23.61 11.306) (width 4.13) (layer F.Cu) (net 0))
 (segment (start 55.544376 11.424522) (end 51.274736 11.424522) (width 4.13) (layer F.Cu) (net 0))
 (segment (start 51.274736 11.424522) (end 47.356794 7.50658) (width 4.13) (layer F.Cu) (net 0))
 (segment (start 51.188851 3.674522) (end 55.544376 3.674522) (width 4.13) (layer F.Cu) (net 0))
 (segment (start 47.356794 7.50658) (end 51.188851 3.674522) (width 4.13) (layer F.Cu) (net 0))
 (segment (start 56.122 3.556) (end 60.39164 3.556) (width 4.13) (layer F.Cu) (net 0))
 (segment (start 64.309582 7.473942) (end 60.477525 11.306) (width 4.13) (layer F.Cu) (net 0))
 (segment (start 60.39164 3.556) (end 64.309582 7.473942) (width 4.13) (layer F.Cu) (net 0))
 (segment (start 60.477525 11.306) (end 56.122 11.306) (width 4.13) (layer F.Cu) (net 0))
 (segment (start 56.122 3.556) (end 56.122 11.306) (width 4.13) (layer F.Cu) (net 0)))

